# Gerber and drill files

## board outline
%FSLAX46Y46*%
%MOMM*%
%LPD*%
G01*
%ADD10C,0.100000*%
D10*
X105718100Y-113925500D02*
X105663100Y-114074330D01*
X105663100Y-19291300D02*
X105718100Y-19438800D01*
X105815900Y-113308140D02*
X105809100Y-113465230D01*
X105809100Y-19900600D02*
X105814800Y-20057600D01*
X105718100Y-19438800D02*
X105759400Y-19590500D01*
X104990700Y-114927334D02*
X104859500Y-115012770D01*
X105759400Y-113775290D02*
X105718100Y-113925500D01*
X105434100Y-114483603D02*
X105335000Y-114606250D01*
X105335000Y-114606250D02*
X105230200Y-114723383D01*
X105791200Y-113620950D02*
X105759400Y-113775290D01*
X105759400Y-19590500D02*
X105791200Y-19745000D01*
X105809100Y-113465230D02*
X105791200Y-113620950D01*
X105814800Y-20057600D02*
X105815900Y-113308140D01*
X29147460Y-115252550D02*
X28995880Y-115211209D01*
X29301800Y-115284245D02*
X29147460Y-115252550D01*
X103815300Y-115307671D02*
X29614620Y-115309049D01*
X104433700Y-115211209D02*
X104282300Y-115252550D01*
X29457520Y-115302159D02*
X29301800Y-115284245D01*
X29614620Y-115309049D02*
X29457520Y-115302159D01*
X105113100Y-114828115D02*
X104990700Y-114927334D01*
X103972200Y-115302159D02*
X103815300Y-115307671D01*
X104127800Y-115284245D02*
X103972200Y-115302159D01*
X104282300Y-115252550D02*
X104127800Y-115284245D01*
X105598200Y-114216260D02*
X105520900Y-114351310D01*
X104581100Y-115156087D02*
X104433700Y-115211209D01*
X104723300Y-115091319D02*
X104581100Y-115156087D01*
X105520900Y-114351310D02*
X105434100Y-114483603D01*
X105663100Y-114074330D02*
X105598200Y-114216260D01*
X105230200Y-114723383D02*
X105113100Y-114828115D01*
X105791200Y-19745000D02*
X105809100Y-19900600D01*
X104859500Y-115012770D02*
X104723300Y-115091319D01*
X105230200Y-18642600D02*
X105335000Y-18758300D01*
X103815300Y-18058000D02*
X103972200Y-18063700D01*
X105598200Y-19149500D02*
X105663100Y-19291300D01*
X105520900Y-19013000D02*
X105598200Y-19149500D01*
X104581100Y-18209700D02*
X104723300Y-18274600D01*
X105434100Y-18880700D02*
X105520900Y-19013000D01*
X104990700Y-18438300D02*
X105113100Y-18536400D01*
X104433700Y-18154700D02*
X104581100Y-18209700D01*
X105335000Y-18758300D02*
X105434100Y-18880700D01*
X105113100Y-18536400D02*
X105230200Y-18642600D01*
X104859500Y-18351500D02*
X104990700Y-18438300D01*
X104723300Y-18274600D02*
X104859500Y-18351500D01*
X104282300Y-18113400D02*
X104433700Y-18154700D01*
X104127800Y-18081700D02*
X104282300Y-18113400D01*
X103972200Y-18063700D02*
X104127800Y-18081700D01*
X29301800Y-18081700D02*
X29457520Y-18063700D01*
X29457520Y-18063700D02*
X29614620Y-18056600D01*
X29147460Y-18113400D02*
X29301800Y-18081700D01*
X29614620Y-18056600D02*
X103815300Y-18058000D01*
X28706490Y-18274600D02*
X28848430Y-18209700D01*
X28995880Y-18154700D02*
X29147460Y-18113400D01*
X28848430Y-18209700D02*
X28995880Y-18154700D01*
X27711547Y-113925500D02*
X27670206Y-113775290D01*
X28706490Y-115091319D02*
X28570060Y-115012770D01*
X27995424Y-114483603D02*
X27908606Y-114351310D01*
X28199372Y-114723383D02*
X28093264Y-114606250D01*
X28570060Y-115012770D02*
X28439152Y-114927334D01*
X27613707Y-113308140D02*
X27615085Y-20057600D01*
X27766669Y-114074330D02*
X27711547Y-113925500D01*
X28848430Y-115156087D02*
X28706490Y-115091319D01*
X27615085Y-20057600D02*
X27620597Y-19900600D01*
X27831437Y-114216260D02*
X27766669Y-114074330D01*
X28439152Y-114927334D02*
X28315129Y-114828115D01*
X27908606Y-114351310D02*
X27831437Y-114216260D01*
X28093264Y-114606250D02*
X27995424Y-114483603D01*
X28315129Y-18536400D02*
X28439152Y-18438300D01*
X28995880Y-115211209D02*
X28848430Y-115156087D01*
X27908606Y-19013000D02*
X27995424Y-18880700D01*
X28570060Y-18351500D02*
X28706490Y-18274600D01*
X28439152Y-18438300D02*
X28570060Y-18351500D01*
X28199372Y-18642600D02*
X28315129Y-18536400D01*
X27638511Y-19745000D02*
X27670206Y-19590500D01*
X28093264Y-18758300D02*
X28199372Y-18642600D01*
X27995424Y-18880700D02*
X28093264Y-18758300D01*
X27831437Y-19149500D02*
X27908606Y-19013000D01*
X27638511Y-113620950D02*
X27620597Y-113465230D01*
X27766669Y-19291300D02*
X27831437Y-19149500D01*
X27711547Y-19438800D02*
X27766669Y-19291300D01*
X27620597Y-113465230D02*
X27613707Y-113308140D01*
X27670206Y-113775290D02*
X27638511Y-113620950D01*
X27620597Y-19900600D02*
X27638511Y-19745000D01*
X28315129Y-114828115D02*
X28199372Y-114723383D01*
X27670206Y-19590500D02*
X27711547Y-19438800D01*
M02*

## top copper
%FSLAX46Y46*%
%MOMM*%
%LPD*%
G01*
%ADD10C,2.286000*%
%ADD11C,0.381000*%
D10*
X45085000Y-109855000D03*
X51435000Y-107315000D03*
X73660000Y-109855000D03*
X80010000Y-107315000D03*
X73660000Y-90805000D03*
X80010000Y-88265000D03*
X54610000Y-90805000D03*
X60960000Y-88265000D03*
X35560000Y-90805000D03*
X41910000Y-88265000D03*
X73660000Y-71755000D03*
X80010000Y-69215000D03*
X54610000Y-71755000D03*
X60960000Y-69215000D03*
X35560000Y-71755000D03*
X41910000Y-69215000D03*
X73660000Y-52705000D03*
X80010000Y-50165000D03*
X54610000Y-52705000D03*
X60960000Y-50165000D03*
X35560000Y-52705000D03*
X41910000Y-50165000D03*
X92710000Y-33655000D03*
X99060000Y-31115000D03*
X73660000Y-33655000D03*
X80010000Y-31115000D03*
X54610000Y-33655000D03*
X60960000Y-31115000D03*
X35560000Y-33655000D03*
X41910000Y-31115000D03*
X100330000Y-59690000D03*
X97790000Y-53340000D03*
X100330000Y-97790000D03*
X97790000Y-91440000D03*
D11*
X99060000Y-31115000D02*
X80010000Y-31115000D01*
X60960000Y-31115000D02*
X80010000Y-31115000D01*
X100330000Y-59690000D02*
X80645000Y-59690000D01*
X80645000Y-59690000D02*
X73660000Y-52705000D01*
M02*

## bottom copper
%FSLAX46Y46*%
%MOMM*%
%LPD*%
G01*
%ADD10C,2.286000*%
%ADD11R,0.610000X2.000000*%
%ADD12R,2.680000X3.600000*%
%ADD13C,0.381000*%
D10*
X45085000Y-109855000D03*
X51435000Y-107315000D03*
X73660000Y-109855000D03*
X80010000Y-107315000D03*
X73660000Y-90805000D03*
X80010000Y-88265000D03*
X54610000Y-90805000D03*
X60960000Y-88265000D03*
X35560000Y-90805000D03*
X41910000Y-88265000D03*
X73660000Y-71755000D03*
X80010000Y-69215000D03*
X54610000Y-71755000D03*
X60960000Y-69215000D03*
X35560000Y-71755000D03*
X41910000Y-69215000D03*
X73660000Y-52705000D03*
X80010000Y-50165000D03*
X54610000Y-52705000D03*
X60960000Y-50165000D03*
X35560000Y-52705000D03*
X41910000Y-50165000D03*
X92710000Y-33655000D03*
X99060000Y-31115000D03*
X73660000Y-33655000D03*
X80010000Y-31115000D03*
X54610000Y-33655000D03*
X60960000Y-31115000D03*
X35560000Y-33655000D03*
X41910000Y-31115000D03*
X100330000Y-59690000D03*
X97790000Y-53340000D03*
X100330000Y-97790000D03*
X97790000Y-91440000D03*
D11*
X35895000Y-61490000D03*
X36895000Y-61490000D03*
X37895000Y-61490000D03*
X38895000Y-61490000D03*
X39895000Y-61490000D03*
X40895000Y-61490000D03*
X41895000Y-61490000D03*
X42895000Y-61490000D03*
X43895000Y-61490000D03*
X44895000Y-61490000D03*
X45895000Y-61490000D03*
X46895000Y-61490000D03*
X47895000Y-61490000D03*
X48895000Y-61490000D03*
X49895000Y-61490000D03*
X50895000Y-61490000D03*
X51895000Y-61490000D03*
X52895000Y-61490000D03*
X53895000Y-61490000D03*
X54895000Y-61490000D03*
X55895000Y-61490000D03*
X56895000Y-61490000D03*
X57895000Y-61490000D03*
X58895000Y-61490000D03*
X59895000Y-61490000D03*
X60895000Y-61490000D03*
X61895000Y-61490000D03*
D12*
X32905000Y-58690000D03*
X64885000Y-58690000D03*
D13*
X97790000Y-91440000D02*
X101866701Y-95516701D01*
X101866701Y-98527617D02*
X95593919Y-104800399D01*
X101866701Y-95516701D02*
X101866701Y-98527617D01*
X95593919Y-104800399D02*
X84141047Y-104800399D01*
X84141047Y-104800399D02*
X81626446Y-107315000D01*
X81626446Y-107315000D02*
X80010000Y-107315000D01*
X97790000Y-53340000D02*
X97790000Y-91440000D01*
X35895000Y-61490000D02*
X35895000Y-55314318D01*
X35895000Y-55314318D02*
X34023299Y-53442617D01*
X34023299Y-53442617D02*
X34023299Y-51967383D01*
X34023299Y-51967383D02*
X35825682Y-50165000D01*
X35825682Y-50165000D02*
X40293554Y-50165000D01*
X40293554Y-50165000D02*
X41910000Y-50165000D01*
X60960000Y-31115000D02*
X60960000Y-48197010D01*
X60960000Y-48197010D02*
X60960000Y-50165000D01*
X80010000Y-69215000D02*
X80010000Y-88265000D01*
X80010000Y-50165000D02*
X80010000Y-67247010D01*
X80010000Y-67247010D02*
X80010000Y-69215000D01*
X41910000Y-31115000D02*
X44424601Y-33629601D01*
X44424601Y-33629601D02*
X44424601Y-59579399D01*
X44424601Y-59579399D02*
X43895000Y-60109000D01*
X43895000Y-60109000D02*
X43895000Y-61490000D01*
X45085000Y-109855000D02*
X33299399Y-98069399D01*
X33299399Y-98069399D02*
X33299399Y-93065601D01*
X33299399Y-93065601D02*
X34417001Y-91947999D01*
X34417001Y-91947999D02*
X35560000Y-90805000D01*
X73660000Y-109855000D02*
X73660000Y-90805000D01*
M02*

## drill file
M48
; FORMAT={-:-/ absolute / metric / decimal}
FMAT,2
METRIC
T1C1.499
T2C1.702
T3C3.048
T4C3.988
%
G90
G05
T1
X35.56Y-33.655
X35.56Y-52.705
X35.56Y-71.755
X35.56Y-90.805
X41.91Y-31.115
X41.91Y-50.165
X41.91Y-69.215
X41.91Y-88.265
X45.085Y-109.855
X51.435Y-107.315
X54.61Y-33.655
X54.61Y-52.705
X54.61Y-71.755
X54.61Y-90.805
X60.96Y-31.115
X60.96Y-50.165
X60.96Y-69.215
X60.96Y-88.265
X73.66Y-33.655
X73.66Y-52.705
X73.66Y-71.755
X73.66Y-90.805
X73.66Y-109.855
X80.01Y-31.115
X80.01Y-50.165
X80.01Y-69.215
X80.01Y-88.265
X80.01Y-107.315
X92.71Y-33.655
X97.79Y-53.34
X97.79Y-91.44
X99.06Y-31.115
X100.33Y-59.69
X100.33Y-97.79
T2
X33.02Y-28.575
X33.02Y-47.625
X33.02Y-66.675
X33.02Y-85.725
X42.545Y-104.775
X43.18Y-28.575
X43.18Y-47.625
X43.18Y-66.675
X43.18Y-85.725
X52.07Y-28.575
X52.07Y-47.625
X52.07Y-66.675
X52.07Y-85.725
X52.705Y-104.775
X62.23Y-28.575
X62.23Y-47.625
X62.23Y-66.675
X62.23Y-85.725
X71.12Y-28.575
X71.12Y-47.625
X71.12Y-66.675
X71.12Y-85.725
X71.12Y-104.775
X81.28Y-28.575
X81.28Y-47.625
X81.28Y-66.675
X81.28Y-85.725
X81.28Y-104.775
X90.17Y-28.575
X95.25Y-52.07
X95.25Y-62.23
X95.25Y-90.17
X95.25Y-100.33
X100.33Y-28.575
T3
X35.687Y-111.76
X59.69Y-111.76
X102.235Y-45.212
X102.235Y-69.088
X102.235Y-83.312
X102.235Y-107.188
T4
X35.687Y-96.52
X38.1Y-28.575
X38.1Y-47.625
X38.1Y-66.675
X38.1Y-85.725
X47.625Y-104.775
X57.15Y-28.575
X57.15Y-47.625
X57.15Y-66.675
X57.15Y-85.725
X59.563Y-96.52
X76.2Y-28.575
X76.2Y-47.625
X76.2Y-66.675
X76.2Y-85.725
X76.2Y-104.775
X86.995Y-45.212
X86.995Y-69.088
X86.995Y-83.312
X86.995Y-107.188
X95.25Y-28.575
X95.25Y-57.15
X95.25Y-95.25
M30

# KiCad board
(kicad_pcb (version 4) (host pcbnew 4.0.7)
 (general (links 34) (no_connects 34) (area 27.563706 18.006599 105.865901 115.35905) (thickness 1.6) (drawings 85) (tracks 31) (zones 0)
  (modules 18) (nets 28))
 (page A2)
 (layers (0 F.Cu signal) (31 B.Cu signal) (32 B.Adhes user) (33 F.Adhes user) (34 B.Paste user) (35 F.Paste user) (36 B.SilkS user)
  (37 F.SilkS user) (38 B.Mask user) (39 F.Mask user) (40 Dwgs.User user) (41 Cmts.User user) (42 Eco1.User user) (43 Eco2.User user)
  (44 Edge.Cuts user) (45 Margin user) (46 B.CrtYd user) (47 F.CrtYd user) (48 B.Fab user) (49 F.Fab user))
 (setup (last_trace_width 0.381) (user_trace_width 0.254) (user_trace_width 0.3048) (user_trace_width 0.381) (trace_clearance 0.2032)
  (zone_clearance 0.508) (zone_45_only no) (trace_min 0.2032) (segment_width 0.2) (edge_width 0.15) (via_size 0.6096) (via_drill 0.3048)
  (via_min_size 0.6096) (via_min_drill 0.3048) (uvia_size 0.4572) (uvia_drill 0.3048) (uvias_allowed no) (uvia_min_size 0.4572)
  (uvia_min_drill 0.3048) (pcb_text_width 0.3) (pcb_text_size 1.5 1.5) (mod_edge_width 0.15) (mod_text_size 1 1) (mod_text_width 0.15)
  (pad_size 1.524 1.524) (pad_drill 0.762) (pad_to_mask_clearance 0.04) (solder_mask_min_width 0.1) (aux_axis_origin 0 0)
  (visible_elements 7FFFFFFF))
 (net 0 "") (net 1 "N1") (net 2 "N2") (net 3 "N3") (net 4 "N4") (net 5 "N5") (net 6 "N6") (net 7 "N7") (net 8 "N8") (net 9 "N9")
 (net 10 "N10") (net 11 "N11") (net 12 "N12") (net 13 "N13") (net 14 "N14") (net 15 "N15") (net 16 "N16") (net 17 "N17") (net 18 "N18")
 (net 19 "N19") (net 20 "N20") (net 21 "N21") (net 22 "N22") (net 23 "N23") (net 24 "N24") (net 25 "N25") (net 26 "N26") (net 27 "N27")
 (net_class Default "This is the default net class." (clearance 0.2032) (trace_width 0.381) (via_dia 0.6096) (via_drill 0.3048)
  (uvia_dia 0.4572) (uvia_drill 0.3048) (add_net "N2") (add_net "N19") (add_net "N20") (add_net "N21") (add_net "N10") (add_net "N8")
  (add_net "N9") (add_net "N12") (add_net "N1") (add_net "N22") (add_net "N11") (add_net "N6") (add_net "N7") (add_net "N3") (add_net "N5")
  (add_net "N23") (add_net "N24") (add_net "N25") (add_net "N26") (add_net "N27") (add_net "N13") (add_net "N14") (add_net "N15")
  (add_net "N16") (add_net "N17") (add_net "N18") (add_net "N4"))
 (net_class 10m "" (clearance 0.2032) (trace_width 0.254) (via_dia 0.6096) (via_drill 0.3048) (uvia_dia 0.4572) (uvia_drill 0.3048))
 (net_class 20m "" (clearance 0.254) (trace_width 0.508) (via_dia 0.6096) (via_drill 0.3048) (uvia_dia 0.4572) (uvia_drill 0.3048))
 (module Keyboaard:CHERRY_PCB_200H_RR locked (layer F.Cu) (at 47.625 104.775)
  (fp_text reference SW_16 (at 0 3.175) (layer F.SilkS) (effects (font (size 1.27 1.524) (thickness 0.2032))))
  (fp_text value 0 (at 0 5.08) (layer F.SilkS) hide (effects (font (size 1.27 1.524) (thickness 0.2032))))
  (pad HOLE np_thru_hole circle (at 0 0) (size 3.9878 3.9878) (drill 3.9878) (layers *.Cu))
  (pad HOLE np_thru_hole circle (at -5.08 0) (size 1.7018 1.7018) (drill 1.7018) (layers *.Cu))
  (pad HOLE np_thru_hole circle (at 5.08 0) (size 1.7018 1.7018) (drill 1.7018) (layers *.Cu))
  (pad HOLE np_thru_hole circle (at -11.938 6.985) (size 3.048 3.048) (drill 3.048) (layers *.Cu))
  (pad HOLE np_thru_hole circle (at 12.065 6.985) (size 3.048 3.048) (drill 3.048) (layers *.Cu))
  (pad HOLE np_thru_hole circle (at -11.938 -8.255) (size 3.9878 3.9878) (drill 3.9878) (layers *.Cu))
  (pad HOLE np_thru_hole circle (at 11.938 -8.255) (size 3.9878 3.9878) (drill 3.9878) (layers *.Cu))
  (pad 1 thru_hole circle (at -2.54 5.08) (size 2.286 2.286) (drill 1.4986) (layers *.Cu *.SilkS *.Mask) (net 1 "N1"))
  (pad 2 thru_hole circle (at 3.81 2.54) (size 2.286 2.286) (drill 1.4986) (layers *.Cu *.SilkS *.Mask) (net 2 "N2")))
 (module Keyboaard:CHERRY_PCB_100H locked (layer F.Cu) (at 76.2 104.775 180)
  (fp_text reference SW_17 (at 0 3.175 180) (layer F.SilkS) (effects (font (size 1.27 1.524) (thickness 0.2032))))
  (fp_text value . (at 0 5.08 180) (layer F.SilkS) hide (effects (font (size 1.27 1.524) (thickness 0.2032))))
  (pad 1 thru_hole circle (at 2.54 -5.08 180) (size 2.286 2.286) (drill 1.4986) (layers *.Cu *.SilkS *.Mask) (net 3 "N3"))
  (pad 2 thru_hole circle (at -3.81 -2.54 180) (size 2.286 2.286) (drill 1.4986) (layers *.Cu *.SilkS *.Mask) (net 2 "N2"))
  (pad HOLE np_thru_hole circle (at 0 0 180) (size 3.9878 3.9878) (drill 3.9878) (layers *.Cu))
  (pad HOLE np_thru_hole circle (at -5.08 0 180) (size 1.7018 1.7018) (drill 1.7018) (layers *.Cu))
  (pad HOLE np_thru_hole circle (at 5.08 0 180) (size 1.7018 1.7018) (drill 1.7018) (layers *.Cu)))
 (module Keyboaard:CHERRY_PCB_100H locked (layer F.Cu) (at 76.2 85.725 180)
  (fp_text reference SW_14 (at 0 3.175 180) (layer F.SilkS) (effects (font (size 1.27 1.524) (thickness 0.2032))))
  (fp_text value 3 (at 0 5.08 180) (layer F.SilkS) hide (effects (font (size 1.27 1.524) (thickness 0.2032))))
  (pad 1 thru_hole circle (at 2.54 -5.08 180) (size 2.286 2.286) (drill 1.4986) (layers *.Cu *.SilkS *.Mask) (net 3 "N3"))
  (pad 2 thru_hole circle (at -3.81 -2.54 180) (size 2.286 2.286) (drill 1.4986) (layers *.Cu *.SilkS *.Mask) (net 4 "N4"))
  (pad HOLE np_thru_hole circle (at 0 0 180) (size 3.9878 3.9878) (drill 3.9878) (layers *.Cu))
  (pad HOLE np_thru_hole circle (at -5.08 0 180) (size 1.7018 1.7018) (drill 1.7018) (layers *.Cu))
  (pad HOLE np_thru_hole circle (at 5.08 0 180) (size 1.7018 1.7018) (drill 1.7018) (layers *.Cu)))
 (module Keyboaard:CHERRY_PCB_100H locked (layer F.Cu) (at 57.15 85.725 180)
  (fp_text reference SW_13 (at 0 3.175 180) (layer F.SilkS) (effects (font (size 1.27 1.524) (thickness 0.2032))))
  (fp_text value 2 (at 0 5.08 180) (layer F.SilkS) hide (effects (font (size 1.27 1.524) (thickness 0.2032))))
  (pad 1 thru_hole circle (at 2.54 -5.08 180) (size 2.286 2.286) (drill 1.4986) (layers *.Cu *.SilkS *.Mask) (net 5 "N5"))
  (pad 2 thru_hole circle (at -3.81 -2.54 180) (size 2.286 2.286) (drill 1.4986) (layers *.Cu *.SilkS *.Mask) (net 4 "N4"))
  (pad HOLE np_thru_hole circle (at 0 0 180) (size 3.9878 3.9878) (drill 3.9878) (layers *.Cu))
  (pad HOLE np_thru_hole circle (at -5.08 0 180) (size 1.7018 1.7018) (drill 1.7018) (layers *.Cu))
  (pad HOLE np_thru_hole circle (at 5.08 0 180) (size 1.7018 1.7018) (drill 1.7018) (layers *.Cu)))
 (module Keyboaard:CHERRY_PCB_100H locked (layer F.Cu) (at 38.1 85.725 180)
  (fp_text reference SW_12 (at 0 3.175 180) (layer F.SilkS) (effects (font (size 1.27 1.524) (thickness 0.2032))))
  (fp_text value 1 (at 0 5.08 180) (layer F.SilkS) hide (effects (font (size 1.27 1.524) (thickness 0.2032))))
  (pad 1 thru_hole circle (at 2.54 -5.08 180) (size 2.286 2.286) (drill 1.4986) (layers *.Cu *.SilkS *.Mask) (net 1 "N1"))
  (pad 2 thru_hole circle (at -3.81 -2.54 180) (size 2.286 2.286) (drill 1.4986) (layers *.Cu *.SilkS *.Mask) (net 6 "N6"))
  (pad HOLE np_thru_hole circle (at 0 0 180) (size 3.9878 3.9878) (drill 3.9878) (layers *.Cu))
  (pad HOLE np_thru_hole circle (at -5.08 0 180) (size 1.7018 1.7018) (drill 1.7018) (layers *.Cu))
  (pad HOLE np_thru_hole circle (at 5.08 0 180) (size 1.7018 1.7018) (drill 1.7018) (layers *.Cu)))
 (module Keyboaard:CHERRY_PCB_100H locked (layer F.Cu) (at 76.2 66.675 180)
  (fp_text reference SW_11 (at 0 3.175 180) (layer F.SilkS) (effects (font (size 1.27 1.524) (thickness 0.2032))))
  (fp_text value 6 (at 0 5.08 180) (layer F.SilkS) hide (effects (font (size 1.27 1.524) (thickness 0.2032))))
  (pad 1 thru_hole circle (at 2.54 -5.08 180) (size 2.286 2.286) (drill 1.4986) (layers *.Cu *.SilkS *.Mask) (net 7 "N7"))
  (pad 2 thru_hole circle (at -3.81 -2.54 180) (size 2.286 2.286) (drill 1.4986) (layers *.Cu *.SilkS *.Mask) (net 4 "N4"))
  (pad HOLE np_thru_hole circle (at 0 0 180) (size 3.9878 3.9878) (drill 3.9878) (layers *.Cu))
  (pad HOLE np_thru_hole circle (at -5.08 0 180) (size 1.7018 1.7018) (drill 1.7018) (layers *.Cu))
  (pad HOLE np_thru_hole circle (at 5.08 0 180) (size 1.7018 1.7018) (drill 1.7018) (layers *.Cu)))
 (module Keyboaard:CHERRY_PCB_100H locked (layer F.Cu) (at 57.15 66.675 180)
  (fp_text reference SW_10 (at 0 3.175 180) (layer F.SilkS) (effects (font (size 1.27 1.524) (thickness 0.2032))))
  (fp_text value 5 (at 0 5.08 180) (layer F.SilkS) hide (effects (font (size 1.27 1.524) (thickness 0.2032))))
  (pad 1 thru_hole circle (at 2.54 -5.08 180) (size 2.286 2.286) (drill 1.4986) (layers *.Cu *.SilkS *.Mask) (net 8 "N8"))
  (pad 2 thru_hole circle (at -3.81 -2.54 180) (size 2.286 2.286) (drill 1.4986) (layers *.Cu *.SilkS *.Mask) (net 2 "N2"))
  (pad HOLE np_thru_hole circle (at 0 0 180) (size 3.9878 3.9878) (drill 3.9878) (layers *.Cu))
  (pad HOLE np_thru_hole circle (at -5.08 0 180) (size 1.7018 1.7018) (drill 1.7018) (layers *.Cu))
  (pad HOLE np_thru_hole circle (at 5.08 0 180) (size 1.7018 1.7018) (drill 1.7018) (layers *.Cu)))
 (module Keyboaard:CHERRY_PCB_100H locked (layer F.Cu) (at 38.1 66.675 180)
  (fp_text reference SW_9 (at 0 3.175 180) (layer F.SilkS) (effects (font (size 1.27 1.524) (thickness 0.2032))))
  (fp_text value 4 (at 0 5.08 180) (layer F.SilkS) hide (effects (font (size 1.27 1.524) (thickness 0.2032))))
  (pad 1 thru_hole circle (at 2.54 -5.08 180) (size 2.286 2.286) (drill 1.4986) (layers *.Cu *.SilkS *.Mask) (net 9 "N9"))
  (pad 2 thru_hole circle (at -3.81 -2.54 180) (size 2.286 2.286) (drill 1.4986) (layers *.Cu *.SilkS *.Mask) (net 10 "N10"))
  (pad HOLE np_thru_hole circle (at 0 0 180) (size 3.9878 3.9878) (drill 3.9878) (layers *.Cu))
  (pad HOLE np_thru_hole circle (at -5.08 0 180) (size 1.7018 1.7018) (drill 1.7018) (layers *.Cu))
  (pad HOLE np_thru_hole circle (at 5.08 0 180) (size 1.7018 1.7018) (drill 1.7018) (layers *.Cu)))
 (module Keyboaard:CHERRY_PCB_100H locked (layer F.Cu) (at 76.2 47.625 180)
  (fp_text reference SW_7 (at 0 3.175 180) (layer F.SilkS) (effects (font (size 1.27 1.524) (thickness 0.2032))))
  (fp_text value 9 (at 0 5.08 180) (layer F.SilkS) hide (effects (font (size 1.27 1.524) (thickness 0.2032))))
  (pad 1 thru_hole circle (at 2.54 -5.08 180) (size 2.286 2.286) (drill 1.4986) (layers *.Cu *.SilkS *.Mask) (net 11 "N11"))
  (pad 2 thru_hole circle (at -3.81 -2.54 180) (size 2.286 2.286) (drill 1.4986) (layers *.Cu *.SilkS *.Mask) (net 4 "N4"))
  (pad HOLE np_thru_hole circle (at 0 0 180) (size 3.9878 3.9878) (drill 3.9878) (layers *.Cu))
  (pad HOLE np_thru_hole circle (at -5.08 0 180) (size 1.7018 1.7018) (drill 1.7018) (layers *.Cu))
  (pad HOLE np_thru_hole circle (at 5.08 0 180) (size 1.7018 1.7018) (drill 1.7018) (layers *.Cu)))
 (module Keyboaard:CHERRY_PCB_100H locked (layer F.Cu) (at 57.15 47.625 180)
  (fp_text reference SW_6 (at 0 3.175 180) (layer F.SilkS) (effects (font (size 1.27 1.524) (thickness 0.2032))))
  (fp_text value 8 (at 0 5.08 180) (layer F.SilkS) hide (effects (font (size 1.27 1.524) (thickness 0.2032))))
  (pad 1 thru_hole circle (at 2.54 -5.08 180) (size 2.286 2.286) (drill 1.4986) (layers *.Cu *.SilkS *.Mask) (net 8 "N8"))
  (pad 2 thru_hole circle (at -3.81 -2.54 180) (size 2.286 2.286) (drill 1.4986) (layers *.Cu *.SilkS *.Mask) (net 6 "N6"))
  (pad HOLE np_thru_hole circle (at 0 0 180) (size 3.9878 3.9878) (drill 3.9878) (layers *.Cu))
  (pad HOLE np_thru_hole circle (at -5.08 0 180) (size 1.7018 1.7018) (drill 1.7018) (layers *.Cu))
  (pad HOLE np_thru_hole circle (at 5.08 0 180) (size 1.7018 1.7018) (drill 1.7018) (layers *.Cu)))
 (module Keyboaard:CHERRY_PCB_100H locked (layer F.Cu) (at 38.1 47.625 180)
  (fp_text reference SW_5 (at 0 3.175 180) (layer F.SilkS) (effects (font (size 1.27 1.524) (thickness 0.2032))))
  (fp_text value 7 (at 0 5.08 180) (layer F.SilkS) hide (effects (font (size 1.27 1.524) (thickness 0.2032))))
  (pad 1 thru_hole circle (at 2.54 -5.08 180) (size 2.286 2.286) (drill 1.4986) (layers *.Cu *.SilkS *.Mask) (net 7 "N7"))
  (pad 2 thru_hole circle (at -3.81 -2.54 180) (size 2.286 2.286) (drill 1.4986) (layers *.Cu *.SilkS *.Mask) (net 2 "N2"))
  (pad HOLE np_thru_hole circle (at 0 0 180) (size 3.9878 3.9878) (drill 3.9878) (layers *.Cu))
  (pad HOLE np_thru_hole circle (at -5.08 0 180) (size 1.7018 1.7018) (drill 1.7018) (layers *.Cu))
  (pad HOLE np_thru_hole circle (at 5.08 0 180) (size 1.7018 1.7018) (drill 1.7018) (layers *.Cu)))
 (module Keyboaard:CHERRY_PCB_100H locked (layer F.Cu) (at 95.25 28.575 180)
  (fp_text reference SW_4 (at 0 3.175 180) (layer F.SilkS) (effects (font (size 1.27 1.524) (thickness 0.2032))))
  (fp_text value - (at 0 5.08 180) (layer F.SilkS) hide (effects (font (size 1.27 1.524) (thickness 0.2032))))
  (pad 1 thru_hole circle (at 2.54 -5.08 180) (size 2.286 2.286) (drill 1.4986) (layers *.Cu *.SilkS *.Mask) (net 7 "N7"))
  (pad 2 thru_hole circle (at -3.81 -2.54 180) (size 2.286 2.286) (drill 1.4986) (layers *.Cu *.SilkS *.Mask) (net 6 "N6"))
  (pad HOLE np_thru_hole circle (at 0 0 180) (size 3.9878 3.9878) (drill 3.9878) (layers *.Cu))
  (pad HOLE np_thru_hole circle (at -5.08 0 180) (size 1.7018 1.7018) (drill 1.7018) (layers *.Cu))
  (pad HOLE np_thru_hole circle (at 5.08 0 180) (size 1.7018 1.7018) (drill 1.7018) (layers *.Cu)))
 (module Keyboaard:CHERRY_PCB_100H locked (layer F.Cu) (at 76.2 28.575 180)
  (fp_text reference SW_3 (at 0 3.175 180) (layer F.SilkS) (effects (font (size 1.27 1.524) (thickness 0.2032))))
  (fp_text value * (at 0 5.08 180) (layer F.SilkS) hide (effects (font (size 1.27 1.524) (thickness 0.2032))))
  (pad 1 thru_hole circle (at 2.54 -5.08 180) (size 2.286 2.286) (drill 1.4986) (layers *.Cu *.SilkS *.Mask) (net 3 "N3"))
  (pad 2 thru_hole circle (at -3.81 -2.54 180) (size 2.286 2.286) (drill 1.4986) (layers *.Cu *.SilkS *.Mask) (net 6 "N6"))
  (pad HOLE np_thru_hole circle (at 0 0 180) (size 3.9878 3.9878) (drill 3.9878) (layers *.Cu))
  (pad HOLE np_thru_hole circle (at -5.08 0 180) (size 1.7018 1.7018) (drill 1.7018) (layers *.Cu))
  (pad HOLE np_thru_hole circle (at 5.08 0 180) (size 1.7018 1.7018) (drill 1.7018) (layers *.Cu)))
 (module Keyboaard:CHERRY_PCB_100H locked (layer F.Cu) (at 57.15 28.575 180)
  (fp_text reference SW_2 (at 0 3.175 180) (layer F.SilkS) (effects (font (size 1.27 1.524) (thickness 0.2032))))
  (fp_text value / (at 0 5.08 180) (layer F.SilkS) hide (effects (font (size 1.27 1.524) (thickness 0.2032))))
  (pad 1 thru_hole circle (at 2.54 -5.08 180) (size 2.286 2.286) (drill 1.4986) (layers *.Cu *.SilkS *.Mask) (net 11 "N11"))
  (pad 2 thru_hole circle (at -3.81 -2.54 180) (size 2.286 2.286) (drill 1.4986) (layers *.Cu *.SilkS *.Mask) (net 6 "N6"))
  (pad HOLE np_thru_hole circle (at 0 0 180) (size 3.9878 3.9878) (drill 3.9878) (layers *.Cu))
  (pad HOLE np_thru_hole circle (at -5.08 0 180) (size 1.7018 1.7018) (drill 1.7018) (layers *.Cu))
  (pad HOLE np_thru_hole circle (at 5.08 0 180) (size 1.7018 1.7018) (drill 1.7018) (layers *.Cu)))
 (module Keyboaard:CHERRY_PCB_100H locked (layer F.Cu) (at 38.1 28.575 180)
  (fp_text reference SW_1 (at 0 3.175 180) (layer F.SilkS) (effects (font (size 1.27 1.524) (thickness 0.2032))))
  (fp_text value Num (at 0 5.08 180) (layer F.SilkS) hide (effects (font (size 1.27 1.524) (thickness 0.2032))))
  (pad 1 thru_hole circle (at 2.54 -5.08 180) (size 2.286 2.286) (drill 1.4986) (layers *.Cu *.SilkS *.Mask) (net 8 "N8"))
  (pad 2 thru_hole circle (at -3.81 -2.54 180) (size 2.286 2.286) (drill 1.4986) (layers *.Cu *.SilkS *.Mask) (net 4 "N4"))
  (pad HOLE np_thru_hole circle (at 0 0 180) (size 3.9878 3.9878) (drill 3.9878) (layers *.Cu))
  (pad HOLE np_thru_hole circle (at -5.08 0 180) (size 1.7018 1.7018) (drill 1.7018) (layers *.Cu))
  (pad HOLE np_thru_hole circle (at 5.08 0 180) (size 1.7018 1.7018) (drill 1.7018) (layers *.Cu)))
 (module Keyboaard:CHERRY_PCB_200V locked (layer F.Cu) (at 95.25 57.15 180)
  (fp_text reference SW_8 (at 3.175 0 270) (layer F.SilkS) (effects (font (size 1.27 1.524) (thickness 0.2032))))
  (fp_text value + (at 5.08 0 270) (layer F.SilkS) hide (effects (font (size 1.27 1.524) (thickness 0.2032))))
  (pad 1 thru_hole circle (at -5.08 -2.54 270) (size 2.286 2.286) (drill 1.4986) (layers *.Cu *.SilkS *.Mask) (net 11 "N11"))
  (pad 2 thru_hole circle (at -2.54 3.81 270) (size 2.286 2.286) (drill 1.4986) (layers *.Cu *.SilkS *.Mask) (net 2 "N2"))
  (pad HOLE np_thru_hole circle (at 0 0 270) (size 3.9878 3.9878) (drill 3.9878) (layers *.Cu))
  (pad HOLE np_thru_hole circle (at 0 5.08 270) (size 1.7018 1.7018) (drill 1.7018) (layers *.Cu))
  (pad HOLE np_thru_hole circle (at 0 -5.08 270) (size 1.7018 1.7018) (drill 1.7018) (layers *.Cu))
  (pad HOLE np_thru_hole circle (at -6.985 11.938 270) (size 3.048 3.048) (drill 3.048) (layers *.Cu))
  (pad HOLE np_thru_hole circle (at -6.985 -11.938 270) (size 3.048 3.048) (drill 3.048) (layers *.Cu))
  (pad HOLE np_thru_hole circle (at 8.255 11.938 270) (size 3.9878 3.9878) (drill 3.9878) (layers *.Cu))
  (pad HOLE np_thru_hole circle (at 8.255 -11.938 270) (size 3.9878 3.9878) (drill 3.9878) (layers *.Cu)))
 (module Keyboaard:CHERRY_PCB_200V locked (layer F.Cu) (at 95.25 95.25 180)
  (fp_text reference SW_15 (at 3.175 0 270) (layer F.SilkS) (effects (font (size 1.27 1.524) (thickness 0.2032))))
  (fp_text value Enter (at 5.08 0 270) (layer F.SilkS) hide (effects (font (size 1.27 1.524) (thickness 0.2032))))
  (pad 1 thru_hole circle (at -5.08 -2.54 270) (size 2.286 2.286) (drill 1.4986) (layers *.Cu *.SilkS *.Mask) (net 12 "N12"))
  (pad 2 thru_hole circle (at -2.54 3.81 270) (size 2.286 2.286) (drill 1.4986) (layers *.Cu *.SilkS *.Mask) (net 2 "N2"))
  (pad HOLE np_thru_hole circle (at 0 0 270) (size 3.9878 3.9878) (drill 3.9878) (layers *.Cu))
  (pad HOLE np_thru_hole circle (at 0 5.08 270) (size 1.7018 1.7018) (drill 1.7018) (layers *.Cu))
  (pad HOLE np_thru_hole circle (at 0 -5.08 270) (size 1.7018 1.7018) (drill 1.7018) (layers *.Cu))
  (pad HOLE np_thru_hole circle (at -6.985 11.938 270) (size 3.048 3.048) (drill 3.048) (layers *.Cu))
  (pad HOLE np_thru_hole circle (at -6.985 -11.938 270) (size 3.048 3.048) (drill 3.048) (layers *.Cu))
  (pad HOLE np_thru_hole circle (at 8.255 11.938 270) (size 3.9878 3.9878) (drill 3.9878) (layers *.Cu))
  (pad HOLE np_thru_hole circle (at 8.255 -11.938 270) (size 3.9878 3.9878) (drill 3.9878) (layers *.Cu)))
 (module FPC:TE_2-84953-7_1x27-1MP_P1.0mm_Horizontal (layer B.Cu) (at 48.895 59.69)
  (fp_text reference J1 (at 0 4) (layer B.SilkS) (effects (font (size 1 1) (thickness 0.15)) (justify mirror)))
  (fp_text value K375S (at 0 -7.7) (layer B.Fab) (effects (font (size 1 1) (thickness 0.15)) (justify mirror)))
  (pad 1 smd rect (at -13 1.8) (size 0.61 2) (layers B.Cu B.Paste B.Mask) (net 2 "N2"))
  (pad 2 smd rect (at -12 1.8) (size 0.61 2) (layers B.Cu B.Paste B.Mask) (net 6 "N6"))
  (pad 3 smd rect (at -11 1.8) (size 0.61 2) (layers B.Cu B.Paste B.Mask) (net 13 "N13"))
  (pad 4 smd rect (at -10 1.8) (size 0.61 2) (layers B.Cu B.Paste B.Mask) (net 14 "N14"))
  (pad 5 smd rect (at -9 1.8) (size 0.61 2) (layers B.Cu B.Paste B.Mask) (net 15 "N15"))
  (pad 6 smd rect (at -8 1.8) (size 0.61 2) (layers B.Cu B.Paste B.Mask) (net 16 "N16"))
  (pad 7 smd rect (at -7 1.8) (size 0.61 2) (layers B.Cu B.Paste B.Mask) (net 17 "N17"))
  (pad 8 smd rect (at -6 1.8) (size 0.61 2) (layers B.Cu B.Paste B.Mask) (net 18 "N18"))
  (pad 9 smd rect (at -5 1.8) (size 0.61 2) (layers B.Cu B.Paste B.Mask) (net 4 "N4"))
  (pad 10 smd rect (at -4 1.8) (size 0.61 2) (layers B.Cu B.Paste B.Mask) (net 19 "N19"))
  (pad 11 smd rect (at -3 1.8) (size 0.61 2) (layers B.Cu B.Paste B.Mask) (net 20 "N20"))
  (pad 12 smd rect (at -2 1.8) (size 0.61 2) (layers B.Cu B.Paste B.Mask) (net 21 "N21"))
  (pad 13 smd rect (at -1 1.8) (size 0.61 2) (layers B.Cu B.Paste B.Mask) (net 10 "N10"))
  (pad 14 smd rect (at 0 1.8) (size 0.61 2) (layers B.Cu B.Paste B.Mask) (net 8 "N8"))
  (pad 15 smd rect (at 1 1.8) (size 0.61 2) (layers B.Cu B.Paste B.Mask) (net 9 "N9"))
  (pad 16 smd rect (at 2 1.8) (size 0.61 2) (layers B.Cu B.Paste B.Mask) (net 12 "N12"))
  (pad 17 smd rect (at 3 1.8) (size 0.61 2) (layers B.Cu B.Paste B.Mask) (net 1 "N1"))
  (pad 18 smd rect (at 4 1.8) (size 0.61 2) (layers B.Cu B.Paste B.Mask) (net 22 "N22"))
  (pad 19 smd rect (at 5 1.8) (size 0.61 2) (layers B.Cu B.Paste B.Mask) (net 11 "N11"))
  (pad 20 smd rect (at 6 1.8) (size 0.61 2) (layers B.Cu B.Paste B.Mask) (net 7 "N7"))
  (pad 21 smd rect (at 7 1.8) (size 0.61 2) (layers B.Cu B.Paste B.Mask) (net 3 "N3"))
  (pad 22 smd rect (at 8 1.8) (size 0.61 2) (layers B.Cu B.Paste B.Mask) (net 5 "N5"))
  (pad 23 smd rect (at 9 1.8) (size 0.61 2) (layers B.Cu B.Paste B.Mask) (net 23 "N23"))
  (pad 24 smd rect (at 10 1.8) (size 0.61 2) (layers B.Cu B.Paste B.Mask) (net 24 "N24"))
  (pad 25 smd rect (at 11 1.8) (size 0.61 2) (layers B.Cu B.Paste B.Mask) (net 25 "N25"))
  (pad 26 smd rect (at 12 1.8) (size 0.61 2) (layers B.Cu B.Paste B.Mask) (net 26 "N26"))
  (pad 27 smd rect (at 13 1.8) (size 0.61 2) (layers B.Cu B.Paste B.Mask) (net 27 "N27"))
  (pad MP smd rect (at -15.99 -1) (size 2.68 3.6) (layers B.Cu B.Paste B.Mask))
  (pad MP smd rect (at 15.99 -1) (size 2.68 3.6) (layers B.Cu B.Paste B.Mask)))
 (gr_line (start 105.7181 113.9255) (end 105.6631 114.07433) (layer Edge.Cuts) (width 0.1))
 (gr_line (start 105.6631 19.2913) (end 105.7181 19.4388) (layer Edge.Cuts) (width 0.1))
 (gr_line (start 105.8159 113.30814) (end 105.8091 113.46523) (layer Edge.Cuts) (width 0.1))
 (gr_line (start 105.8091 19.9006) (end 105.8148 20.0576) (layer Edge.Cuts) (width 0.1))
 (gr_line (start 105.7181 19.4388) (end 105.7594 19.5905) (layer Edge.Cuts) (width 0.1))
 (gr_line (start 104.9907 114.927334) (end 104.8595 115.01277) (layer Edge.Cuts) (width 0.1))
 (gr_line (start 105.7594 113.77529) (end 105.7181 113.9255) (layer Edge.Cuts) (width 0.1))
 (gr_line (start 105.4341 114.483603) (end 105.335 114.60625) (layer Edge.Cuts) (width 0.1))
 (gr_line (start 105.335 114.60625) (end 105.2302 114.723383) (layer Edge.Cuts) (width 0.1))
 (gr_line (start 105.7912 113.62095) (end 105.7594 113.77529) (layer Edge.Cuts) (width 0.1))
 (gr_line (start 105.7594 19.5905) (end 105.7912 19.745) (layer Edge.Cuts) (width 0.1))
 (gr_line (start 105.8091 113.46523) (end 105.7912 113.62095) (layer Edge.Cuts) (width 0.1))
 (gr_line (start 105.8148 20.0576) (end 105.8159 113.30814) (layer Edge.Cuts) (width 0.1))
 (gr_line (start 29.14746 115.25255) (end 28.99588 115.211209) (layer Edge.Cuts) (width 0.1))
 (gr_line (start 29.3018 115.284245) (end 29.14746 115.25255) (layer Edge.Cuts) (width 0.1))
 (gr_line (start 103.8153 115.307671) (end 29.61462 115.309049) (layer Edge.Cuts) (width 0.1))
 (gr_line (start 104.4337 115.211209) (end 104.2823 115.25255) (layer Edge.Cuts) (width 0.1))
 (gr_line (start 29.45752 115.302159) (end 29.3018 115.284245) (layer Edge.Cuts) (width 0.1))
 (gr_line (start 29.61462 115.309049) (end 29.45752 115.302159) (layer Edge.Cuts) (width 0.1))
 (gr_line (start 105.1131 114.828115) (end 104.9907 114.927334) (layer Edge.Cuts) (width 0.1))
 (gr_line (start 103.9722 115.302159) (end 103.8153 115.307671) (layer Edge.Cuts) (width 0.1))
 (gr_line (start 104.1278 115.284245) (end 103.9722 115.302159) (layer Edge.Cuts) (width 0.1))
 (gr_line (start 104.2823 115.25255) (end 104.1278 115.284245) (layer Edge.Cuts) (width 0.1))
 (gr_line (start 105.5982 114.21626) (end 105.5209 114.35131) (layer Edge.Cuts) (width 0.1))
 (gr_line (start 104.5811 115.156087) (end 104.4337 115.211209) (layer Edge.Cuts) (width 0.1))
 (gr_line (start 104.7233 115.091319) (end 104.5811 115.156087) (layer Edge.Cuts) (width 0.1))
 (gr_line (start 105.5209 114.35131) (end 105.4341 114.483603) (layer Edge.Cuts) (width 0.1))
 (gr_line (start 105.6631 114.07433) (end 105.5982 114.21626) (layer Edge.Cuts) (width 0.1))
 (gr_line (start 105.2302 114.723383) (end 105.1131 114.828115) (layer Edge.Cuts) (width 0.1))
 (gr_line (start 105.7912 19.745) (end 105.8091 19.9006) (layer Edge.Cuts) (width 0.1))
 (gr_line (start 104.8595 115.01277) (end 104.7233 115.091319) (layer Edge.Cuts) (width 0.1))
 (gr_line (start 105.2302 18.6426) (end 105.335 18.7583) (layer Edge.Cuts) (width 0.1))
 (gr_line (start 103.8153 18.058) (end 103.9722 18.0637) (layer Edge.Cuts) (width 0.1))
 (gr_line (start 105.5982 19.1495) (end 105.6631 19.2913) (layer Edge.Cuts) (width 0.1))
 (gr_line (start 105.5209 19.013) (end 105.5982 19.1495) (layer Edge.Cuts) (width 0.1))
 (gr_line (start 104.5811 18.2097) (end 104.7233 18.2746) (layer Edge.Cuts) (width 0.1))
 (gr_line (start 105.4341 18.8807) (end 105.5209 19.013) (layer Edge.Cuts) (width 0.1))
 (gr_line (start 104.9907 18.4383) (end 105.1131 18.5364) (layer Edge.Cuts) (width 0.1))
 (gr_line (start 104.4337 18.1547) (end 104.5811 18.2097) (layer Edge.Cuts) (width 0.1))
 (gr_line (start 105.335 18.7583) (end 105.4341 18.8807) (layer Edge.Cuts) (width 0.1))
 (gr_line (start 105.1131 18.5364) (end 105.2302 18.6426) (layer Edge.Cuts) (width 0.1))
 (gr_line (start 104.8595 18.3515) (end 104.9907 18.4383) (layer Edge.Cuts) (width 0.1))
 (gr_line (start 104.7233 18.2746) (end 104.8595 18.3515) (layer Edge.Cuts) (width 0.1))
 (gr_line (start 104.2823 18.1134) (end 104.4337 18.1547) (layer Edge.Cuts) (width 0.1))
 (gr_line (start 104.1278 18.0817) (end 104.2823 18.1134) (layer Edge.Cuts) (width 0.1))
 (gr_line (start 103.9722 18.0637) (end 104.1278 18.0817) (layer Edge.Cuts) (width 0.1))
 (gr_line (start 29.3018 18.0817) (end 29.45752 18.0637) (layer Edge.Cuts) (width 0.1))
 (gr_line (start 29.45752 18.0637) (end 29.61462 18.0566) (layer Edge.Cuts) (width 0.1))
 (gr_line (start 29.14746 18.1134) (end 29.3018 18.0817) (layer Edge.Cuts) (width 0.1))
 (gr_line (start 29.61462 18.0566) (end 103.8153 18.058) (layer Edge.Cuts) (width 0.1))
 (gr_line (start 28.70649 18.2746) (end 28.84843 18.2097) (layer Edge.Cuts) (width 0.1))
 (gr_line (start 28.99588 18.1547) (end 29.14746 18.1134) (layer Edge.Cuts) (width 0.1))
 (gr_line (start 28.84843 18.2097) (end 28.99588 18.1547) (layer Edge.Cuts) (width 0.1))
 (gr_line (start 27.711547 113.9255) (end 27.670206 113.77529) (layer Edge.Cuts) (width 0.1))
 (gr_line (start 28.70649 115.091319) (end 28.57006 115.01277) (layer Edge.Cuts) (width 0.1))
 (gr_line (start 27.995424 114.483603) (end 27.908606 114.35131) (layer Edge.Cuts) (width 0.1))
 (gr_line (start 28.199372 114.723383) (end 28.093264 114.60625) (layer Edge.Cuts) (width 0.1))
 (gr_line (start 28.57006 115.01277) (end 28.439152 114.927334) (layer Edge.Cuts) (width 0.1))
 (gr_line (start 27.613707 113.30814) (end 27.615085 20.0576) (layer Edge.Cuts) (width 0.1))
 (gr_line (start 27.766669 114.07433) (end 27.711547 113.9255) (layer Edge.Cuts) (width 0.1))
 (gr_line (start 28.84843 115.156087) (end 28.70649 115.091319) (layer Edge.Cuts) (width 0.1))
 (gr_line (start 27.615085 20.0576) (end 27.620597 19.9006) (layer Edge.Cuts) (width 0.1))
 (gr_line (start 27.831437 114.21626) (end 27.766669 114.07433) (layer Edge.Cuts) (width 0.1))
 (gr_line (start 28.439152 114.927334) (end 28.315129 114.828115) (layer Edge.Cuts) (width 0.1))
 (gr_line (start 27.908606 114.35131) (end 27.831437 114.21626) (layer Edge.Cuts) (width 0.1))
 (gr_line (start 28.093264 114.60625) (end 27.995424 114.483603) (layer Edge.Cuts) (width 0.1))
 (gr_line (start 28.315129 18.5364) (end 28.439152 18.4383) (layer Edge.Cuts) (width 0.1))
 (gr_line (start 28.99588 115.211209) (end 28.84843 115.156087) (layer Edge.Cuts) (width 0.1))
 (gr_line (start 27.908606 19.013) (end 27.995424 18.8807) (layer Edge.Cuts) (width 0.1))
 (gr_line (start 28.57006 18.3515) (end 28.70649 18.2746) (layer Edge.Cuts) (width 0.1))
 (gr_line (start 28.439152 18.4383) (end 28.57006 18.3515) (layer Edge.Cuts) (width 0.1))
 (gr_line (start 28.199372 18.6426) (end 28.315129 18.5364) (layer Edge.Cuts) (width 0.1))
 (gr_line (start 27.638511 19.745) (end 27.670206 19.5905) (layer Edge.Cuts) (width 0.1))
 (gr_line (start 28.093264 18.7583) (end 28.199372 18.6426) (layer Edge.Cuts) (width 0.1))
 (gr_line (start 27.995424 18.8807) (end 28.093264 18.7583) (layer Edge.Cuts) (width 0.1))
 (gr_line (start 27.831437 19.1495) (end 27.908606 19.013) (layer Edge.Cuts) (width 0.1))
 (gr_line (start 27.638511 113.62095) (end 27.620597 113.46523) (layer Edge.Cuts) (width 0.1))
 (gr_line (start 27.766669 19.2913) (end 27.831437 19.1495) (layer Edge.Cuts) (width 0.1))
 (gr_line (start 27.711547 19.4388) (end 27.766669 19.2913) (layer Edge.Cuts) (width 0.1))
 (gr_line (start 27.620597 113.46523) (end 27.613707 113.30814) (layer Edge.Cuts) (width 0.1))
 (gr_line (start 27.670206 113.77529) (end 27.638511 113.62095) (layer Edge.Cuts) (width 0.1))
 (gr_line (start 27.620597 19.9006) (end 27.638511 19.745) (layer Edge.Cuts) (width 0.1))
 (gr_line (start 28.315129 114.828115) (end 28.199372 114.723383) (layer Edge.Cuts) (width 0.1))
 (gr_line (start 27.670206 19.5905) (end 27.711547 19.4388) (layer Edge.Cuts) (width 0.1))
 (segment (start 97.79 91.44) (end 101.866701 95.516701) (width 0.381) (layer B.Cu) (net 2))
 (segment (start 101.866701 98.527617) (end 95.593919 104.800399) (width 0.381) (layer B.Cu) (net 2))
 (segment (start 101.866701 95.516701) (end 101.866701 98.527617) (width 0.381) (layer B.Cu) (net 2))
 (segment (start 95.593919 104.800399) (end 84.141047 104.800399) (width 0.381) (layer B.Cu) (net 2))
 (segment (start 84.141047 104.800399) (end 81.626446 107.315) (width 0.381) (layer B.Cu) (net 2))
 (segment (start 81.626446 107.315) (end 80.01 107.315) (width 0.381) (layer B.Cu) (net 2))
 (segment (start 97.79 53.34) (end 97.79 91.44) (width 0.381) (layer B.Cu) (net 2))
 (segment (start 35.895 61.49) (end 35.895 55.314318) (width 0.381) (layer B.Cu) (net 2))
 (segment (start 35.895 55.314318) (end 34.023299 53.442617) (width 0.381) (layer B.Cu) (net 2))
 (segment (start 34.023299 53.442617) (end 34.023299 51.967383) (width 0.381) (layer B.Cu) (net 2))
 (segment (start 34.023299 51.967383) (end 35.825682 50.165) (width 0.381) (layer B.Cu) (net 2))
 (segment (start 35.825682 50.165) (end 40.293554 50.165) (width 0.381) (layer B.Cu) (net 2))
 (segment (start 40.293554 50.165) (end 41.91 50.165) (width 0.381) (layer B.Cu) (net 2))
 (segment (start 60.96 31.115) (end 60.96 48.19701) (width 0.381) (layer B.Cu) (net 6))
 (segment (start 60.96 48.19701) (end 60.96 50.165) (width 0.381) (layer B.Cu) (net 6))
 (segment (start 99.06 31.115) (end 80.01 31.115) (width 0.381) (layer F.Cu) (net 6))
 (segment (start 60.96 31.115) (end 80.01 31.115) (width 0.381) (layer F.Cu) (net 6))
 (segment (start 80.01 69.215) (end 80.01 88.265) (width 0.381) (layer B.Cu) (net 4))
 (segment (start 80.01 50.165) (end 80.01 67.24701) (width 0.381) (layer B.Cu) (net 4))
 (segment (start 80.01 67.24701) (end 80.01 69.215) (width 0.381) (layer B.Cu) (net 4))
 (segment (start 41.91 31.115) (end 44.424601 33.629601) (width 0.381) (layer B.Cu) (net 4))
 (segment (start 44.424601 33.629601) (end 44.424601 59.579399) (width 0.381) (layer B.Cu) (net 4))
 (segment (start 44.424601 59.579399) (end 43.895 60.109) (width 0.381) (layer B.Cu) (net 4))
 (segment (start 43.895 60.109) (end 43.895 61.49) (width 0.381) (layer B.Cu) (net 4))
 (segment (start 45.085 109.855) (end 33.299399 98.069399) (width 0.381) (layer B.Cu) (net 1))
 (segment (start 33.299399 98.069399) (end 33.299399 93.065601) (width 0.381) (layer B.Cu) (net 1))
 (segment (start 33.299399 93.065601) (end 34.417001 91.947999) (width 0.381) (layer B.Cu) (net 1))
 (segment (start 34.417001 91.947999) (end 35.56 90.805) (width 0.381) (layer B.Cu) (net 1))
 (segment (start 100.33 59.69) (end 80.645 59.69) (width 0.381) (layer F.Cu) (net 11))
 (segment (start 80.645 59.69) (end 73.66 52.705) (width 0.381) (layer F.Cu) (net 11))
 (segment (start 73.66 109.855) (end 73.66 90.805) (width 0.381) (layer B.Cu) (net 3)))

